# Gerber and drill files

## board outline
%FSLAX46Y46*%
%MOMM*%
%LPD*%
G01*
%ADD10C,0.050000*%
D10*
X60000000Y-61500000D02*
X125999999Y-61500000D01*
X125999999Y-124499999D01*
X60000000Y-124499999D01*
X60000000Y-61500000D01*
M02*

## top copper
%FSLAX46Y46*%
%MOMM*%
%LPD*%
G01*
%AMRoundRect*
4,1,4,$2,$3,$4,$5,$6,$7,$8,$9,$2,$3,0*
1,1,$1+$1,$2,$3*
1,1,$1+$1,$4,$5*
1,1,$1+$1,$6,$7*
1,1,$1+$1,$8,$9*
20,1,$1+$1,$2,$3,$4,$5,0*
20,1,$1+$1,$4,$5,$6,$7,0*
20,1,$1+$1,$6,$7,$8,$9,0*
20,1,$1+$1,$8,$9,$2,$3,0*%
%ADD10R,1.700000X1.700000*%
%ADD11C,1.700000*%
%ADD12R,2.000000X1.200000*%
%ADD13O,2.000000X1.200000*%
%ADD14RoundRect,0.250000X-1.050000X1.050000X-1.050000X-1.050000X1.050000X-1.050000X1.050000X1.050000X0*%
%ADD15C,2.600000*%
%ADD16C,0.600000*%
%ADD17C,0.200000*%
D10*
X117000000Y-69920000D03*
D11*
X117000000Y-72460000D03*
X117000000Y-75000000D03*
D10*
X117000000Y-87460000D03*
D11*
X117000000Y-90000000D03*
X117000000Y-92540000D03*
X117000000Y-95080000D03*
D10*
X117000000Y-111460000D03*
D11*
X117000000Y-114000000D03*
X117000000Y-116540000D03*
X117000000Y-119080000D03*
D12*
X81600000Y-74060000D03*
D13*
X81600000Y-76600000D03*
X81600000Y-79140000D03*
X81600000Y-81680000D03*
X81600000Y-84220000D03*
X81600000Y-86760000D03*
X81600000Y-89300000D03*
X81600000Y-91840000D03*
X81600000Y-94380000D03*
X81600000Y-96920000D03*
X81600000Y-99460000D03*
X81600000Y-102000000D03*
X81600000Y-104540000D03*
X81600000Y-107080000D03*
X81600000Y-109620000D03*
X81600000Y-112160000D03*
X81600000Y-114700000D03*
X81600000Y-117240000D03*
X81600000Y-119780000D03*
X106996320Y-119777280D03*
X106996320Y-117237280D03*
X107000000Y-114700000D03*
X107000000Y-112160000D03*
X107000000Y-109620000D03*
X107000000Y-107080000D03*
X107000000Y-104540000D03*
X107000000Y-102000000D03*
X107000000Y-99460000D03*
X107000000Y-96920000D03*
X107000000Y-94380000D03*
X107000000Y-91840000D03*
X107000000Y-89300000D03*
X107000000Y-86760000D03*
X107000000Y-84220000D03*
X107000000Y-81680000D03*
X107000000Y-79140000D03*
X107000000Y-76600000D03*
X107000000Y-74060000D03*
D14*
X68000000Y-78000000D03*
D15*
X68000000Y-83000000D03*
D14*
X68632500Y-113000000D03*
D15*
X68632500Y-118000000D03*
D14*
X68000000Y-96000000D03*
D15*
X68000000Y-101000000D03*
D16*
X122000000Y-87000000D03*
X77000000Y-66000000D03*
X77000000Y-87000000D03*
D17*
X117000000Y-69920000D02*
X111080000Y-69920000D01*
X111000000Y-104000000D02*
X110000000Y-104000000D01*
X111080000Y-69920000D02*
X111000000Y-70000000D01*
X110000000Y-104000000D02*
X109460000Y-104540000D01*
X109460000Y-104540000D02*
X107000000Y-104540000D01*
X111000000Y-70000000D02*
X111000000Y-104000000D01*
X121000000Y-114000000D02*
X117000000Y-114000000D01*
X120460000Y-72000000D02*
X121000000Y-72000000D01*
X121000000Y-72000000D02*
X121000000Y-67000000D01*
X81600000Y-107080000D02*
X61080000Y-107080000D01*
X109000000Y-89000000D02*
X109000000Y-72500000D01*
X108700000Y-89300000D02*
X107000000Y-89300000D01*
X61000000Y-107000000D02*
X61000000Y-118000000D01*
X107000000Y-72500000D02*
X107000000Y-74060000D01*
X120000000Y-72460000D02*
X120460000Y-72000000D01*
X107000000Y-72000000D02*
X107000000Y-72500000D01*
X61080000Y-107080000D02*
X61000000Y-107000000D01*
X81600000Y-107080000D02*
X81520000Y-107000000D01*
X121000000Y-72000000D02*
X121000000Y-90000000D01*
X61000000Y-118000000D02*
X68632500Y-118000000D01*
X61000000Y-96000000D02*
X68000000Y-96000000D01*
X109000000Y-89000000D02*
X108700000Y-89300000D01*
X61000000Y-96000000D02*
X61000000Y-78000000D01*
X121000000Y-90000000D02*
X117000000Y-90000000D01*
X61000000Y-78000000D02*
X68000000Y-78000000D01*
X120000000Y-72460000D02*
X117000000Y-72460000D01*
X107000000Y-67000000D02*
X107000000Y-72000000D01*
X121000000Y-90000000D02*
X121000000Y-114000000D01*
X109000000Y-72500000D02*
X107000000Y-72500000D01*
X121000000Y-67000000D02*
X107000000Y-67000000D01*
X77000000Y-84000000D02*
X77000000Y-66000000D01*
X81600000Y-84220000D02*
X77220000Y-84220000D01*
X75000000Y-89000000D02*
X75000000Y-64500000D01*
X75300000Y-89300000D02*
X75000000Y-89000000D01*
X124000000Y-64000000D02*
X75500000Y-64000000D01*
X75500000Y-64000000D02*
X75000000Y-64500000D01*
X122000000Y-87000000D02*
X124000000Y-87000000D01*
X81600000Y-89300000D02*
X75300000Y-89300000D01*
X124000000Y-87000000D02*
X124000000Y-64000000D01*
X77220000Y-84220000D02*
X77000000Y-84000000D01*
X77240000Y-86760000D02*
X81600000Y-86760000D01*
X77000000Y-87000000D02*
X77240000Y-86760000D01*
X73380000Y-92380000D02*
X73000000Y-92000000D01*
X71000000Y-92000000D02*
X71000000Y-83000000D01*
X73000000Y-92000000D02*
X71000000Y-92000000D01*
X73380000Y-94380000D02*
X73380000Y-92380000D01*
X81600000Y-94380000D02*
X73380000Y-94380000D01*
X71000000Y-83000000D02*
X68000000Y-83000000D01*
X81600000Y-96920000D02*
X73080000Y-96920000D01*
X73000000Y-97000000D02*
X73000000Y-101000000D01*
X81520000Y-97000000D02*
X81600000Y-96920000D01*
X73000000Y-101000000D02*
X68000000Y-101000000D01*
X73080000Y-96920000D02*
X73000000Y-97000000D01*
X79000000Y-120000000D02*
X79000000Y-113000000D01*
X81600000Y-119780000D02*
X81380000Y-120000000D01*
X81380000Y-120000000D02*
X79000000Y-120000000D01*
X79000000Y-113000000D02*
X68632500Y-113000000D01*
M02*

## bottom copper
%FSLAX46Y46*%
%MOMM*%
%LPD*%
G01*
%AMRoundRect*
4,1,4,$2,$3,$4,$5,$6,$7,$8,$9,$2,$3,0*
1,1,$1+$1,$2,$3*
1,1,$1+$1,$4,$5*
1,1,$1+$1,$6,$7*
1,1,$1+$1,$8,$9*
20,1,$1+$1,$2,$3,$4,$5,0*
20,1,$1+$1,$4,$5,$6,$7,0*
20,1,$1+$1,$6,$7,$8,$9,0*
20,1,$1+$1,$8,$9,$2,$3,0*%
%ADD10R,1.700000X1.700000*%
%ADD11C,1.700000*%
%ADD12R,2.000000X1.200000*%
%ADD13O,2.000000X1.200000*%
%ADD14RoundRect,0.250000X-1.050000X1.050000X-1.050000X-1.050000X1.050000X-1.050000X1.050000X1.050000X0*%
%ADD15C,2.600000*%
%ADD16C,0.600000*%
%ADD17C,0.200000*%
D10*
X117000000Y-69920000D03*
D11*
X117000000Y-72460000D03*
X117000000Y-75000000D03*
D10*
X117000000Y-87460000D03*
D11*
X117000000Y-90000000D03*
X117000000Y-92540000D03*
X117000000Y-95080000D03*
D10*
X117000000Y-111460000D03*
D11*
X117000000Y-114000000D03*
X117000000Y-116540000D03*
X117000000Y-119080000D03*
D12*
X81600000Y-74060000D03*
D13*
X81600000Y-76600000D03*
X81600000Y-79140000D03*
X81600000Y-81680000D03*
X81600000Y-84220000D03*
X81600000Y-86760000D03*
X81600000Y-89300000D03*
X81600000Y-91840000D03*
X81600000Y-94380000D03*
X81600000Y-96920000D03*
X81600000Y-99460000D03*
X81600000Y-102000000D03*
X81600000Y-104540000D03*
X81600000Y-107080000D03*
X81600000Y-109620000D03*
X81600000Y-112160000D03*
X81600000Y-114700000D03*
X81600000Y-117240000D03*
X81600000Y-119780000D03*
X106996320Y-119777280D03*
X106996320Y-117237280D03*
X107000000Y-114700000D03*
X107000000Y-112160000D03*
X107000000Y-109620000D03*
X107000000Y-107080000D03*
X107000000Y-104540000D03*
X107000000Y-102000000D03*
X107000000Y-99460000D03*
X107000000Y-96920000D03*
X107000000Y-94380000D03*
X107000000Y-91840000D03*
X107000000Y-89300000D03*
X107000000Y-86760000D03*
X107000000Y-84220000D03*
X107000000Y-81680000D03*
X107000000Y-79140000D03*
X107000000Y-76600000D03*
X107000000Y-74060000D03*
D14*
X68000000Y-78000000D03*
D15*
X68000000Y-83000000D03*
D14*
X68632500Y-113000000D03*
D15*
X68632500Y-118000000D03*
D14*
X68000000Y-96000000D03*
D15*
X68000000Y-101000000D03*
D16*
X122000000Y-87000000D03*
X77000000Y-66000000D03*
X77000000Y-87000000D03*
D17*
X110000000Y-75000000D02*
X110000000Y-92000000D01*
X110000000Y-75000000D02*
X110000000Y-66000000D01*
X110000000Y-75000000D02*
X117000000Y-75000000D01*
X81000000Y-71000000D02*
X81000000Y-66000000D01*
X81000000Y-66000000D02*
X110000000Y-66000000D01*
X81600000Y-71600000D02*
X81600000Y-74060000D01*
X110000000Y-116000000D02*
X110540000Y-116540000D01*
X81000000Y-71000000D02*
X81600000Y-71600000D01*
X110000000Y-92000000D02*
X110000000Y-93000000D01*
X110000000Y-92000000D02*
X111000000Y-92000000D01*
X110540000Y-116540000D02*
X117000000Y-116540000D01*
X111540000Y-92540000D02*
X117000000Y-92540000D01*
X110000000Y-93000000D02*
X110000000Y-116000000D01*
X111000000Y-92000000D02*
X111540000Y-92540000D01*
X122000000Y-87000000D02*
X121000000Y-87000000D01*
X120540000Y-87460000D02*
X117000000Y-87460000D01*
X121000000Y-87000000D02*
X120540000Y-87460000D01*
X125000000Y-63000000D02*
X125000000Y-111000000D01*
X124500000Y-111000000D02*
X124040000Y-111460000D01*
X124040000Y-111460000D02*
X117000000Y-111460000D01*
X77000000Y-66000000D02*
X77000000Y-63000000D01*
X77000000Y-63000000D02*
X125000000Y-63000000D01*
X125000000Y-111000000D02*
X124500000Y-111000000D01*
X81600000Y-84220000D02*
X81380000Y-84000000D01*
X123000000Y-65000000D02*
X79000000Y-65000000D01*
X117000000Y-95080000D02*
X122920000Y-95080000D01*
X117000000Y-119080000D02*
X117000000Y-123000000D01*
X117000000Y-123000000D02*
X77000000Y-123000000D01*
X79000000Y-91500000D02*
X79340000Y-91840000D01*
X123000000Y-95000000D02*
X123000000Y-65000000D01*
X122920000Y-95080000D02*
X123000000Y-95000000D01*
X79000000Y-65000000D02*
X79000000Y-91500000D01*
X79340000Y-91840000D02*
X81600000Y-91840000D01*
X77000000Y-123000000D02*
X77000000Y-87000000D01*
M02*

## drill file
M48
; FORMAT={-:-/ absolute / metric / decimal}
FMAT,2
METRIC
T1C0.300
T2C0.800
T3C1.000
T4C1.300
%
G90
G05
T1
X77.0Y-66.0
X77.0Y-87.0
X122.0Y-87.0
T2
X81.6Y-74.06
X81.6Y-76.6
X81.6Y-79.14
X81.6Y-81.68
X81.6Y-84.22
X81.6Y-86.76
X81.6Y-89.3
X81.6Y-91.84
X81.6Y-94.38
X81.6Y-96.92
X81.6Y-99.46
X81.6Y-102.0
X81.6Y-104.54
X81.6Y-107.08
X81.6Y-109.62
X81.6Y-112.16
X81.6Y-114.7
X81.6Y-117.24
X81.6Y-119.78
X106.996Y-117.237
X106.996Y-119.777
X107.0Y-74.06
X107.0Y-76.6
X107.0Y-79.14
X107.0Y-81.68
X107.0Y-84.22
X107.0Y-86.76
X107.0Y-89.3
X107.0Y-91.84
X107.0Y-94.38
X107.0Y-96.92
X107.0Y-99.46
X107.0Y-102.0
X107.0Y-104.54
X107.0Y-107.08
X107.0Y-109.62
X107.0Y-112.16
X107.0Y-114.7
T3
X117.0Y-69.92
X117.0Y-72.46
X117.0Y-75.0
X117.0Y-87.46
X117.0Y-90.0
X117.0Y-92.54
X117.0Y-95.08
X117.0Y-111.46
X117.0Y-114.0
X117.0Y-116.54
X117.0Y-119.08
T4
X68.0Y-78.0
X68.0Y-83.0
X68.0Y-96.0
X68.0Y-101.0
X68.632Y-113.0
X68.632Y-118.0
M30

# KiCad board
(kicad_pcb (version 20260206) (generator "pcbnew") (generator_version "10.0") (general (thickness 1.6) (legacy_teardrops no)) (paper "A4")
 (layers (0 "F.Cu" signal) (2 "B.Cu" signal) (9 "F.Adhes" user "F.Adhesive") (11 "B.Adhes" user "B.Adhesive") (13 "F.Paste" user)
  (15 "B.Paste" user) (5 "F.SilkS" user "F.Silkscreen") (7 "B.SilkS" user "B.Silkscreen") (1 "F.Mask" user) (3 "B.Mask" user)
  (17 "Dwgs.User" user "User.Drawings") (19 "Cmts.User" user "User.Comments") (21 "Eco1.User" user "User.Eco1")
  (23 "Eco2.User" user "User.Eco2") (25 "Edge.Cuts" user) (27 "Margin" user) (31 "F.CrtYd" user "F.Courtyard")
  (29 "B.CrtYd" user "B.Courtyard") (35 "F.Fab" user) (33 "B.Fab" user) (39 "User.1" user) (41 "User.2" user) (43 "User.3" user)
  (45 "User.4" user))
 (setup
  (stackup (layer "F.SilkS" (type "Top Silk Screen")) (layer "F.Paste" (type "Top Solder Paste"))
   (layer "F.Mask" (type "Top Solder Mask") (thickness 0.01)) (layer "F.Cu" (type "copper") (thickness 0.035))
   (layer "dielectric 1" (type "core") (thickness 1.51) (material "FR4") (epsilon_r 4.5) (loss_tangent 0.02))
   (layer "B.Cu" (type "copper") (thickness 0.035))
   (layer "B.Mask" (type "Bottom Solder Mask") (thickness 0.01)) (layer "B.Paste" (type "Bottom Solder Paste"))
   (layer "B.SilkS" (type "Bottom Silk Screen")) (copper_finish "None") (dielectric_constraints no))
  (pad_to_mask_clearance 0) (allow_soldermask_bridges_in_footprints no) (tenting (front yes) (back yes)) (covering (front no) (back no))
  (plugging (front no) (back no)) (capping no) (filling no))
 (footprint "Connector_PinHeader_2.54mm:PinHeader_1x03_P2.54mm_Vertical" (layer "F.Cu") (at 117 69.92)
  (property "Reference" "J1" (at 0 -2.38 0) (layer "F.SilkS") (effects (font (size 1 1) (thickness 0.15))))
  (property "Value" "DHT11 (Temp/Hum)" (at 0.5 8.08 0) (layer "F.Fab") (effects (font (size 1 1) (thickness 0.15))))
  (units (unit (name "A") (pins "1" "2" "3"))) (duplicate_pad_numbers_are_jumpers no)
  (pad "1" thru_hole rect (at 0 0) (size 1.7 1.7) (drill 1) (layers "*.Cu" "*.Mask") (remove_unused_layers no) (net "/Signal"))
  (pad "2" thru_hole circle (at 0 2.54) (size 1.7 1.7) (drill 1) (layers "*.Cu" "*.Mask") (remove_unused_layers no) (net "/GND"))
  (pad "3" thru_hole circle (at 0 5.08) (size 1.7 1.7) (drill 1) (layers "*.Cu" "*.Mask") (remove_unused_layers no) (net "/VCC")))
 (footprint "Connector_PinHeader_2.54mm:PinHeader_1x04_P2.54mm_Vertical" (layer "F.Cu") (at 117 87.46)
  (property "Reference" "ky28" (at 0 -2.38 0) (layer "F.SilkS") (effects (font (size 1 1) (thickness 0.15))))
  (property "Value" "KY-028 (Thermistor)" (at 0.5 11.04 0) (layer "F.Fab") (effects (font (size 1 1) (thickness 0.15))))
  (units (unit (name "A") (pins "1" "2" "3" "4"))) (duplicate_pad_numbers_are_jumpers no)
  (pad "1" thru_hole rect (at 0 0) (size 1.7 1.7) (drill 1) (layers "*.Cu" "*.Mask") (remove_unused_layers no) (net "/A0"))
  (pad "2" thru_hole circle (at 0 2.54) (size 1.7 1.7) (drill 1) (layers "*.Cu" "*.Mask") (remove_unused_layers no) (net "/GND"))
  (pad "3" thru_hole circle (at 0 5.08) (size 1.7 1.7) (drill 1) (layers "*.Cu" "*.Mask") (remove_unused_layers no) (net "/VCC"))
  (pad "4" thru_hole circle (at 0 7.62) (size 1.7 1.7) (drill 1) (layers "*.Cu" "*.Mask") (remove_unused_layers no) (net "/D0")))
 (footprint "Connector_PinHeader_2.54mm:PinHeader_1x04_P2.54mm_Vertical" (layer "F.Cu") (at 117 111.46)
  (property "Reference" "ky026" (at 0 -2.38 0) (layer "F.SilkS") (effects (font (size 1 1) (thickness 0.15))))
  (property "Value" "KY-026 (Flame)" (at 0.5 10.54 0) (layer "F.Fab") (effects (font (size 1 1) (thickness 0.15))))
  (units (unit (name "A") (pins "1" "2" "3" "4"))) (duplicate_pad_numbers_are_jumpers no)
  (pad "1" thru_hole rect (at 0 0) (size 1.7 1.7) (drill 1) (layers "*.Cu" "*.Mask") (remove_unused_layers no) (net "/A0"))
  (pad "2" thru_hole circle (at 0 2.54) (size 1.7 1.7) (drill 1) (layers "*.Cu" "*.Mask") (remove_unused_layers no) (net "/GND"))
  (pad "3" thru_hole circle (at 0 5.08) (size 1.7 1.7) (drill 1) (layers "*.Cu" "*.Mask") (remove_unused_layers no) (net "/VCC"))
  (pad "4" thru_hole circle (at 0 7.62) (size 1.7 1.7) (drill 1) (layers "*.Cu" "*.Mask") (remove_unused_layers no) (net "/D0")))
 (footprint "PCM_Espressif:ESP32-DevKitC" (layer "F.Cu") (at 81.6 74.06)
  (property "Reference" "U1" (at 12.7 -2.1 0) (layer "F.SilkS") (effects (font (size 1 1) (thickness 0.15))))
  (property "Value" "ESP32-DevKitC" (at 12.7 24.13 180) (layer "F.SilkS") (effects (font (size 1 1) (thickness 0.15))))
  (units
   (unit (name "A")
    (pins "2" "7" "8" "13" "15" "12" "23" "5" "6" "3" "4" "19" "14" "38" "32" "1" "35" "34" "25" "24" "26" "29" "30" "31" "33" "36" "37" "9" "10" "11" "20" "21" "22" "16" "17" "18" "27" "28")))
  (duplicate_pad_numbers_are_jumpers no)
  (pad "1" thru_hole rect (at 0 0 270) (size 1.2 2) (drill 0.8) (layers "*.Cu" "*.Mask") (remove_unused_layers no) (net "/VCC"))
  (pad "2" thru_hole oval (at 0 2.54 270) (size 1.2 2) (drill 0.8) (layers "*.Cu" "*.Mask") (remove_unused_layers no)
   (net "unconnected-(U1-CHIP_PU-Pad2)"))
  (pad "3" thru_hole oval (at 0 5.08 270) (size 1.2 2) (drill 0.8) (layers "*.Cu" "*.Mask") (remove_unused_layers no)
   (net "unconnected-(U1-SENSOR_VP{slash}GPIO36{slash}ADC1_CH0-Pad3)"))
  (pad "4" thru_hole oval (at 0 7.62 270) (size 1.2 2) (drill 0.8) (layers "*.Cu" "*.Mask") (remove_unused_layers no)
   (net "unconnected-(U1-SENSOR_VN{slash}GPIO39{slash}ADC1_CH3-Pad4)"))
  (pad "5" thru_hole oval (at 0 10.16 270) (size 1.2 2) (drill 0.8) (layers "*.Cu" "*.Mask") (remove_unused_layers no) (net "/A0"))
  (pad "6" thru_hole oval (at 0 12.7 270) (size 1.2 2) (drill 0.8) (layers "*.Cu" "*.Mask") (remove_unused_layers no) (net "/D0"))
  (pad "7" thru_hole oval (at 0 15.24 270) (size 1.2 2) (drill 0.8) (layers "*.Cu" "*.Mask") (remove_unused_layers no) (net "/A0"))
  (pad "8" thru_hole oval (at 0 17.78 270) (size 1.2 2) (drill 0.8) (layers "*.Cu" "*.Mask") (remove_unused_layers no) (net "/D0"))
  (pad "9" thru_hole oval (at 0 20.32 270) (size 1.2 2) (drill 0.8) (layers "*.Cu" "*.Mask") (remove_unused_layers no)
   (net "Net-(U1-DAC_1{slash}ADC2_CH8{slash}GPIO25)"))
  (pad "10" thru_hole oval (at 0 22.86 270) (size 1.2 2) (drill 0.8) (layers "*.Cu" "*.Mask") (remove_unused_layers no)
   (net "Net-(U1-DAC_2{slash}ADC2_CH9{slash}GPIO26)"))
  (pad "11" thru_hole oval (at 0 25.4 270) (size 1.2 2) (drill 0.8) (layers "*.Cu" "*.Mask") (remove_unused_layers no)
   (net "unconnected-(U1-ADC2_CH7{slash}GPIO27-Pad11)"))
  (pad "12" thru_hole oval (at 0 27.94 270) (size 1.2 2) (drill 0.8) (layers "*.Cu" "*.Mask") (remove_unused_layers no)
   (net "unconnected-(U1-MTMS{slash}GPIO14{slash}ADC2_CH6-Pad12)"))
  (pad "13" thru_hole oval (at 0 30.48 270) (size 1.2 2) (drill 0.8) (layers "*.Cu" "*.Mask") (remove_unused_layers no)
   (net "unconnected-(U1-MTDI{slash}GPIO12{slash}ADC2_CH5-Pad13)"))
  (pad "14" thru_hole oval (at 0 33.02 270) (size 1.2 2) (drill 0.8) (layers "*.Cu" "*.Mask") (remove_unused_layers no) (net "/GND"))
  (pad "15" thru_hole oval (at 0 35.56 270) (size 1.2 2) (drill 0.8) (layers "*.Cu" "*.Mask") (remove_unused_layers no)
   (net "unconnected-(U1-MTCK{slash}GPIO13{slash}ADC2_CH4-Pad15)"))
  (pad "16" thru_hole oval (at 0 38.1 270) (size 1.2 2) (drill 0.8) (layers "*.Cu" "*.Mask") (remove_unused_layers no)
   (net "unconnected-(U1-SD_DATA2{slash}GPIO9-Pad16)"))
  (pad "17" thru_hole oval (at 0 40.64 270) (size 1.2 2) (drill 0.8) (layers "*.Cu" "*.Mask") (remove_unused_layers no)
   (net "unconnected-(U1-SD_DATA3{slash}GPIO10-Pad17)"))
  (pad "18" thru_hole oval (at 0 43.18 270) (size 1.2 2) (drill 0.8) (layers "*.Cu" "*.Mask") (remove_unused_layers no)
   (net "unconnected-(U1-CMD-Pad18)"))
  (pad "19" thru_hole oval (at 0 45.72 270) (size 1.2 2) (drill 0.8) (layers "*.Cu" "*.Mask") (remove_unused_layers no) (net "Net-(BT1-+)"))
  (pad "20" thru_hole oval (at 25.39632 45.71728 270) (size 1.2 2) (drill 0.8) (layers "*.Cu" "*.Mask") (remove_unused_layers no)
   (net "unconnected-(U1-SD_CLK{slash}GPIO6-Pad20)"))
  (pad "21" thru_hole oval (at 25.39632 43.17728 270) (size 1.2 2) (drill 0.8) (layers "*.Cu" "*.Mask") (remove_unused_layers no)
   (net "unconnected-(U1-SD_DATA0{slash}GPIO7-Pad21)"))
  (pad "22" thru_hole oval (at 25.4 40.64 270) (size 1.2 2) (drill 0.8) (layers "*.Cu" "*.Mask") (remove_unused_layers no)
   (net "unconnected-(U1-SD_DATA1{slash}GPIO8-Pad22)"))
  (pad "23" thru_hole oval (at 25.4 38.1 270) (size 1.2 2) (drill 0.8) (layers "*.Cu" "*.Mask") (remove_unused_layers no)
   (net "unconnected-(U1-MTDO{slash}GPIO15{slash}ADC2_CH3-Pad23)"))
  (pad "24" thru_hole oval (at 25.4 35.56 270) (size 1.2 2) (drill 0.8) (layers "*.Cu" "*.Mask") (remove_unused_layers no)
   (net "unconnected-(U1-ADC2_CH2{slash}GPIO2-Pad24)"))
  (pad "25" thru_hole oval (at 25.4 33.02 270) (size 1.2 2) (drill 0.8) (layers "*.Cu" "*.Mask") (remove_unused_layers no)
   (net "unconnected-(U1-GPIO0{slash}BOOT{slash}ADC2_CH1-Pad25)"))
  (pad "26" thru_hole oval (at 25.4 30.48 270) (size 1.2 2) (drill 0.8) (layers "*.Cu" "*.Mask") (remove_unused_layers no) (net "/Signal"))
  (pad "27" thru_hole oval (at 25.4 27.94 270) (size 1.2 2) (drill 0.8) (layers "*.Cu" "*.Mask") (remove_unused_layers no)
   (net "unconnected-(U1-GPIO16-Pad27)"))
  (pad "28" thru_hole oval (at 25.4 25.4 270) (size 1.2 2) (drill 0.8) (layers "*.Cu" "*.Mask") (remove_unused_layers no)
   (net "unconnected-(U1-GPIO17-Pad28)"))
  (pad "29" thru_hole oval (at 25.4 22.86 270) (size 1.2 2) (drill 0.8) (layers "*.Cu" "*.Mask") (remove_unused_layers no)
   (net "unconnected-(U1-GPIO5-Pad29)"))
  (pad "30" thru_hole oval (at 25.4 20.32 270) (size 1.2 2) (drill 0.8) (layers "*.Cu" "*.Mask") (remove_unused_layers no)
   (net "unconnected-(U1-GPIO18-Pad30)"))
  (pad "31" thru_hole oval (at 25.4 17.78 270) (size 1.2 2) (drill 0.8) (layers "*.Cu" "*.Mask") (remove_unused_layers no)
   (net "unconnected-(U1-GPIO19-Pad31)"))
  (pad "32" thru_hole oval (at 25.4 15.24 270) (size 1.2 2) (drill 0.8) (layers "*.Cu" "*.Mask") (remove_unused_layers no) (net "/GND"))
  (pad "33" thru_hole oval (at 25.4 12.7 270) (size 1.2 2) (drill 0.8) (layers "*.Cu" "*.Mask") (remove_unused_layers no)
   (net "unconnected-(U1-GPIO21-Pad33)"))
  (pad "34" thru_hole oval (at 25.4 10.16 270) (size 1.2 2) (drill 0.8) (layers "*.Cu" "*.Mask") (remove_unused_layers no)
   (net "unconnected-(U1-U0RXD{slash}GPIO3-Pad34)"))
  (pad "35" thru_hole oval (at 25.4 7.62 270) (size 1.2 2) (drill 0.8) (layers "*.Cu" "*.Mask") (remove_unused_layers no)
   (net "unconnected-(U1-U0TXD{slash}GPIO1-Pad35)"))
  (pad "36" thru_hole oval (at 25.4 5.08 270) (size 1.2 2) (drill 0.8) (layers "*.Cu" "*.Mask") (remove_unused_layers no)
   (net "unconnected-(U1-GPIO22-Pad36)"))
  (pad "37" thru_hole oval (at 25.4 2.54 270) (size 1.2 2) (drill 0.8) (layers "*.Cu" "*.Mask") (remove_unused_layers no)
   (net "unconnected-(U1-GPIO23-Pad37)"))
  (pad "38" thru_hole oval (at 25.4 0 270) (size 1.2 2) (drill 0.8) (layers "*.Cu" "*.Mask") (remove_unused_layers no) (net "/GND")))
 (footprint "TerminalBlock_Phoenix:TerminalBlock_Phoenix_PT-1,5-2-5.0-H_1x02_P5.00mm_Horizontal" (layer "F.Cu") (at 68 78 -90)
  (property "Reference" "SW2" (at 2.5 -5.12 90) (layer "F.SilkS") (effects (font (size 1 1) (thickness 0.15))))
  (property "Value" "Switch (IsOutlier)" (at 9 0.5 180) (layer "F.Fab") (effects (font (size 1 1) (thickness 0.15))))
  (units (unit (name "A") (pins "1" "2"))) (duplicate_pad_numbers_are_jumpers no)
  (pad "1" thru_hole roundrect (at 0 0 270) (size 2.6 2.6) (drill 1.3) (layers "*.Cu" "*.Mask") (remove_unused_layers no)
   (roundrect_rratio 0.096154) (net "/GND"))
  (pad "2" thru_hole circle (at 5 0 270) (size 2.6 2.6) (drill 1.3) (layers "*.Cu" "*.Mask") (remove_unused_layers no)
   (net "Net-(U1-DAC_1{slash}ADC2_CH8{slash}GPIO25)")))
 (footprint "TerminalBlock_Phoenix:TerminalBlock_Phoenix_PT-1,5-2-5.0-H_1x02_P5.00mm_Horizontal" (layer "F.Cu") (at 68.6325 113 -90)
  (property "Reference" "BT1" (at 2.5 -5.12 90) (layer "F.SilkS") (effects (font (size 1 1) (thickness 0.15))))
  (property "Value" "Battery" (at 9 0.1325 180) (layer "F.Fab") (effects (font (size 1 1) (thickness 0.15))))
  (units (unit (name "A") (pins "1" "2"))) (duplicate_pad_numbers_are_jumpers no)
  (pad "1" thru_hole roundrect (at 0 0 270) (size 2.6 2.6) (drill 1.3) (layers "*.Cu" "*.Mask") (remove_unused_layers no)
   (roundrect_rratio 0.096154) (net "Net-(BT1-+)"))
  (pad "2" thru_hole circle (at 5 0 270) (size 2.6 2.6) (drill 1.3) (layers "*.Cu" "*.Mask") (remove_unused_layers no) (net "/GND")))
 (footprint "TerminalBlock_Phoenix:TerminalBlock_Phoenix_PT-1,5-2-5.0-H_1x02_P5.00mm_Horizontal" (layer "F.Cu") (at 68 96 -90)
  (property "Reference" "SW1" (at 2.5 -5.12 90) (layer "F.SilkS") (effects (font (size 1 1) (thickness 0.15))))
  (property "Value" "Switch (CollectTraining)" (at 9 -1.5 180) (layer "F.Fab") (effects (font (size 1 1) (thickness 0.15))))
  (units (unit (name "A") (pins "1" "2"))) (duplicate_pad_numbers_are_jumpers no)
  (pad "1" thru_hole roundrect (at 0 0 270) (size 2.6 2.6) (drill 1.3) (layers "*.Cu" "*.Mask") (remove_unused_layers no)
   (roundrect_rratio 0.096154) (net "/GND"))
  (pad "2" thru_hole circle (at 5 0 270) (size 2.6 2.6) (drill 1.3) (layers "*.Cu" "*.Mask") (remove_unused_layers no)
   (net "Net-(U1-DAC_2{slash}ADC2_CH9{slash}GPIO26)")))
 (gr_rect (start 60 61.5) (end 125.999999 124.499999) (stroke (width 0.05) (type default)) (fill no) (layer "Edge.Cuts"))
 (segment (start 117 69.92) (end 111.08 69.92) (width 0.2) (layer "F.Cu") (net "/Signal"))
 (segment (start 111 104) (end 110 104) (width 0.2) (layer "F.Cu") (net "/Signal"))
 (segment (start 111.08 69.92) (end 111 70) (width 0.2) (layer "F.Cu") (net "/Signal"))
 (segment (start 110 104) (end 109.46 104.54) (width 0.2) (layer "F.Cu") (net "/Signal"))
 (segment (start 109.46 104.54) (end 107 104.54) (width 0.2) (layer "F.Cu") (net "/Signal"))
 (segment (start 111 70) (end 111 104) (width 0.2) (layer "F.Cu") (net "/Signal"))
 (segment (start 121 114) (end 117 114) (width 0.2) (layer "F.Cu") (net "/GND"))
 (segment (start 120.46 72) (end 121 72) (width 0.2) (layer "F.Cu") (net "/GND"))
 (segment (start 121 72) (end 121 67) (width 0.2) (layer "F.Cu") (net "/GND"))
 (segment (start 81.6 107.08) (end 61.08 107.08) (width 0.2) (layer "F.Cu") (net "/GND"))
 (segment (start 109 89) (end 109 72.5) (width 0.2) (layer "F.Cu") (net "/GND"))
 (segment (start 108.7 89.3) (end 107 89.3) (width 0.2) (layer "F.Cu") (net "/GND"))
 (segment (start 61 107) (end 61 118) (width 0.2) (layer "F.Cu") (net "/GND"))
 (segment (start 107 72.5) (end 107 74.06) (width 0.2) (layer "F.Cu") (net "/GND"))
 (segment (start 120 72.46) (end 120.46 72) (width 0.2) (layer "F.Cu") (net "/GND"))
 (segment (start 107 72) (end 107 72.5) (width 0.2) (layer "F.Cu") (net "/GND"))
 (segment (start 61.08 107.08) (end 61 107) (width 0.2) (layer "F.Cu") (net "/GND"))
 (segment (start 81.6 107.08) (end 81.52 107) (width 0.2) (layer "F.Cu") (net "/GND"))
 (segment (start 121 72) (end 121 90) (width 0.2) (layer "F.Cu") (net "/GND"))
 (segment (start 61 118) (end 68.6325 118) (width 0.2) (layer "F.Cu") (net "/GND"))
 (segment (start 61 96) (end 68 96) (width 0.2) (layer "F.Cu") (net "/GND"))
 (segment (start 109 89) (end 108.7 89.3) (width 0.2) (layer "F.Cu") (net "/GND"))
 (segment (start 61 96) (end 61 78) (width 0.2) (layer "F.Cu") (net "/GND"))
 (segment (start 121 90) (end 117 90) (width 0.2) (layer "F.Cu") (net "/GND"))
 (segment (start 61 78) (end 68 78) (width 0.2) (layer "F.Cu") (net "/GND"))
 (segment (start 120 72.46) (end 117 72.46) (width 0.2) (layer "F.Cu") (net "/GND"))
 (segment (start 107 67) (end 107 72) (width 0.2) (layer "F.Cu") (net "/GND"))
 (segment (start 121 90) (end 121 114) (width 0.2) (layer "F.Cu") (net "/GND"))
 (segment (start 109 72.5) (end 107 72.5) (width 0.2) (layer "F.Cu") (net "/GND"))
 (segment (start 121 67) (end 107 67) (width 0.2) (layer "F.Cu") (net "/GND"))
 (segment (start 110 75) (end 110 92) (width 0.2) (layer "B.Cu") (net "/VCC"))
 (segment (start 110 75) (end 110 66) (width 0.2) (layer "B.Cu") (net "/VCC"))
 (segment (start 110 75) (end 117 75) (width 0.2) (layer "B.Cu") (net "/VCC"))
 (segment (start 81 71) (end 81 66) (width 0.2) (layer "B.Cu") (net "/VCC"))
 (segment (start 81 66) (end 110 66) (width 0.2) (layer "B.Cu") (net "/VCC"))
 (segment (start 81.6 71.6) (end 81.6 74.06) (width 0.2) (layer "B.Cu") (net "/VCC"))
 (segment (start 110 116) (end 110.54 116.54) (width 0.2) (layer "B.Cu") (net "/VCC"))
 (segment (start 81 71) (end 81.6 71.6) (width 0.2) (layer "B.Cu") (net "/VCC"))
 (segment (start 110 92) (end 110 93) (width 0.2) (layer "B.Cu") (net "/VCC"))
 (segment (start 110 92) (end 111 92) (width 0.2) (layer "B.Cu") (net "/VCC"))
 (segment (start 110.54 116.54) (end 117 116.54) (width 0.2) (layer "B.Cu") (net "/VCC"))
 (segment (start 111.54 92.54) (end 117 92.54) (width 0.2) (layer "B.Cu") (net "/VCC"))
 (segment (start 110 93) (end 110 116) (width 0.2) (layer "B.Cu") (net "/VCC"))
 (segment (start 111 92) (end 111.54 92.54) (width 0.2) (layer "B.Cu") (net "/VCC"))
 (segment (start 77 84) (end 77 66) (width 0.2) (layer "F.Cu") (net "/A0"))
 (segment (start 81.6 84.22) (end 77.22 84.22) (width 0.2) (layer "F.Cu") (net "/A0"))
 (segment (start 75 89) (end 75 64.5) (width 0.2) (layer "F.Cu") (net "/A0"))
 (segment (start 75.3 89.3) (end 75 89) (width 0.2) (layer "F.Cu") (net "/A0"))
 (segment (start 124 64) (end 75.5 64) (width 0.2) (layer "F.Cu") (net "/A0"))
 (segment (start 75.5 64) (end 75 64.5) (width 0.2) (layer "F.Cu") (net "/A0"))
 (segment (start 122 87) (end 124 87) (width 0.2) (layer "F.Cu") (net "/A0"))
 (segment (start 81.6 89.3) (end 75.3 89.3) (width 0.2) (layer "F.Cu") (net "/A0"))
 (segment (start 124 87) (end 124 64) (width 0.2) (layer "F.Cu") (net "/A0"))
 (segment (start 77.22 84.22) (end 77 84) (width 0.2) (layer "F.Cu") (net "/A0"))
 (via (at 122 87) (size 0.6) (drill 0.3) (layers "F.Cu" "B.Cu") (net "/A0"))
 (via (at 77 66) (size 0.6) (drill 0.3) (layers "F.Cu" "B.Cu") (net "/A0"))
 (segment (start 122 87) (end 121 87) (width 0.2) (layer "B.Cu") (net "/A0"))
 (segment (start 120.54 87.46) (end 117 87.46) (width 0.2) (layer "B.Cu") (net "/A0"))
 (segment (start 121 87) (end 120.54 87.46) (width 0.2) (layer "B.Cu") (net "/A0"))
 (segment (start 125 63) (end 125 111) (width 0.2) (layer "B.Cu") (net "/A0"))
 (segment (start 124.5 111) (end 124.04 111.46) (width 0.2) (layer "B.Cu") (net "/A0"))
 (segment (start 124.04 111.46) (end 117 111.46) (width 0.2) (layer "B.Cu") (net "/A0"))
 (segment (start 77 66) (end 77 63) (width 0.2) (layer "B.Cu") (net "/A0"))
 (segment (start 77 63) (end 125 63) (width 0.2) (layer "B.Cu") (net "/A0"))
 (segment (start 125 111) (end 124.5 111) (width 0.2) (layer "B.Cu") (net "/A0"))
 (segment (start 81.6 84.22) (end 81.38 84) (width 0.2) (layer "B.Cu") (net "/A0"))
 (segment (start 77.24 86.76) (end 81.6 86.76) (width 0.2) (layer "F.Cu") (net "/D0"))
 (segment (start 77 87) (end 77.24 86.76) (width 0.2) (layer "F.Cu") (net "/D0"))
 (via (at 77 87) (size 0.6) (drill 0.3) (layers "F.Cu" "B.Cu") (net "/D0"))
 (segment (start 123 65) (end 79 65) (width 0.2) (layer "B.Cu") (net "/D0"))
 (segment (start 117 95.08) (end 122.92 95.08) (width 0.2) (layer "B.Cu") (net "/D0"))
 (segment (start 117 119.08) (end 117 123) (width 0.2) (layer "B.Cu") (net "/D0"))
 (segment (start 117 123) (end 77 123) (width 0.2) (layer "B.Cu") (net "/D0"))
 (segment (start 79 91.5) (end 79.34 91.84) (width 0.2) (layer "B.Cu") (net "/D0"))
 (segment (start 123 95) (end 123 65) (width 0.2) (layer "B.Cu") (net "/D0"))
 (segment (start 122.92 95.08) (end 123 95) (width 0.2) (layer "B.Cu") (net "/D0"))
 (segment (start 79 65) (end 79 91.5) (width 0.2) (layer "B.Cu") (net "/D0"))
 (segment (start 79.34 91.84) (end 81.6 91.84) (width 0.2) (layer "B.Cu") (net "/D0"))
 (segment (start 77 123) (end 77 87) (width 0.2) (layer "B.Cu") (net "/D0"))
 (segment (start 73.38 92.38) (end 73 92) (width 0.2) (layer "F.Cu") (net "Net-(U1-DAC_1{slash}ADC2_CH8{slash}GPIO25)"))
 (segment (start 71 92) (end 71 83) (width 0.2) (layer "F.Cu") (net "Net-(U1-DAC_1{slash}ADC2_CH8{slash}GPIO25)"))
 (segment (start 73 92) (end 71 92) (width 0.2) (layer "F.Cu") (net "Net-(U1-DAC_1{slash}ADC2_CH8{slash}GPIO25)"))
 (segment (start 73.38 94.38) (end 73.38 92.38) (width 0.2) (layer "F.Cu") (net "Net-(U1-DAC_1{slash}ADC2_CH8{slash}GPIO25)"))
 (segment (start 81.6 94.38) (end 73.38 94.38) (width 0.2) (layer "F.Cu") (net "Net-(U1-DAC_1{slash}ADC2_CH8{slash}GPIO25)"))
 (segment (start 71 83) (end 68 83) (width 0.2) (layer "F.Cu") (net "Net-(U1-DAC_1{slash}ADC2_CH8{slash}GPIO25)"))
 (segment (start 81.6 96.92) (end 73.08 96.92) (width 0.2) (layer "F.Cu") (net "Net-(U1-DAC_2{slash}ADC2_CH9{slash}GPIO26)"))
 (segment (start 73 97) (end 73 101) (width 0.2) (layer "F.Cu") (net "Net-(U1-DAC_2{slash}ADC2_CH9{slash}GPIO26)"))
 (segment (start 81.52 97) (end 81.6 96.92) (width 0.2) (layer "F.Cu") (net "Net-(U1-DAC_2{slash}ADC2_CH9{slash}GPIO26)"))
 (segment (start 73 101) (end 68 101) (width 0.2) (layer "F.Cu") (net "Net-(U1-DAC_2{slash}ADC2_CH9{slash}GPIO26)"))
 (segment (start 73.08 96.92) (end 73 97) (width 0.2) (layer "F.Cu") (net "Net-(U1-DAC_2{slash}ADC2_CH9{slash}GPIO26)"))
 (segment (start 79 120) (end 79 113) (width 0.2) (layer "F.Cu") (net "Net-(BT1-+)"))
 (segment (start 81.6 119.78) (end 81.38 120) (width 0.2) (layer "F.Cu") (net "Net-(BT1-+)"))
 (segment (start 81.38 120) (end 79 120) (width 0.2) (layer "F.Cu") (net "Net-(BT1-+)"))
 (segment (start 79 113) (end 68.6325 113) (width 0.2) (layer "F.Cu") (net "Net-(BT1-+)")))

